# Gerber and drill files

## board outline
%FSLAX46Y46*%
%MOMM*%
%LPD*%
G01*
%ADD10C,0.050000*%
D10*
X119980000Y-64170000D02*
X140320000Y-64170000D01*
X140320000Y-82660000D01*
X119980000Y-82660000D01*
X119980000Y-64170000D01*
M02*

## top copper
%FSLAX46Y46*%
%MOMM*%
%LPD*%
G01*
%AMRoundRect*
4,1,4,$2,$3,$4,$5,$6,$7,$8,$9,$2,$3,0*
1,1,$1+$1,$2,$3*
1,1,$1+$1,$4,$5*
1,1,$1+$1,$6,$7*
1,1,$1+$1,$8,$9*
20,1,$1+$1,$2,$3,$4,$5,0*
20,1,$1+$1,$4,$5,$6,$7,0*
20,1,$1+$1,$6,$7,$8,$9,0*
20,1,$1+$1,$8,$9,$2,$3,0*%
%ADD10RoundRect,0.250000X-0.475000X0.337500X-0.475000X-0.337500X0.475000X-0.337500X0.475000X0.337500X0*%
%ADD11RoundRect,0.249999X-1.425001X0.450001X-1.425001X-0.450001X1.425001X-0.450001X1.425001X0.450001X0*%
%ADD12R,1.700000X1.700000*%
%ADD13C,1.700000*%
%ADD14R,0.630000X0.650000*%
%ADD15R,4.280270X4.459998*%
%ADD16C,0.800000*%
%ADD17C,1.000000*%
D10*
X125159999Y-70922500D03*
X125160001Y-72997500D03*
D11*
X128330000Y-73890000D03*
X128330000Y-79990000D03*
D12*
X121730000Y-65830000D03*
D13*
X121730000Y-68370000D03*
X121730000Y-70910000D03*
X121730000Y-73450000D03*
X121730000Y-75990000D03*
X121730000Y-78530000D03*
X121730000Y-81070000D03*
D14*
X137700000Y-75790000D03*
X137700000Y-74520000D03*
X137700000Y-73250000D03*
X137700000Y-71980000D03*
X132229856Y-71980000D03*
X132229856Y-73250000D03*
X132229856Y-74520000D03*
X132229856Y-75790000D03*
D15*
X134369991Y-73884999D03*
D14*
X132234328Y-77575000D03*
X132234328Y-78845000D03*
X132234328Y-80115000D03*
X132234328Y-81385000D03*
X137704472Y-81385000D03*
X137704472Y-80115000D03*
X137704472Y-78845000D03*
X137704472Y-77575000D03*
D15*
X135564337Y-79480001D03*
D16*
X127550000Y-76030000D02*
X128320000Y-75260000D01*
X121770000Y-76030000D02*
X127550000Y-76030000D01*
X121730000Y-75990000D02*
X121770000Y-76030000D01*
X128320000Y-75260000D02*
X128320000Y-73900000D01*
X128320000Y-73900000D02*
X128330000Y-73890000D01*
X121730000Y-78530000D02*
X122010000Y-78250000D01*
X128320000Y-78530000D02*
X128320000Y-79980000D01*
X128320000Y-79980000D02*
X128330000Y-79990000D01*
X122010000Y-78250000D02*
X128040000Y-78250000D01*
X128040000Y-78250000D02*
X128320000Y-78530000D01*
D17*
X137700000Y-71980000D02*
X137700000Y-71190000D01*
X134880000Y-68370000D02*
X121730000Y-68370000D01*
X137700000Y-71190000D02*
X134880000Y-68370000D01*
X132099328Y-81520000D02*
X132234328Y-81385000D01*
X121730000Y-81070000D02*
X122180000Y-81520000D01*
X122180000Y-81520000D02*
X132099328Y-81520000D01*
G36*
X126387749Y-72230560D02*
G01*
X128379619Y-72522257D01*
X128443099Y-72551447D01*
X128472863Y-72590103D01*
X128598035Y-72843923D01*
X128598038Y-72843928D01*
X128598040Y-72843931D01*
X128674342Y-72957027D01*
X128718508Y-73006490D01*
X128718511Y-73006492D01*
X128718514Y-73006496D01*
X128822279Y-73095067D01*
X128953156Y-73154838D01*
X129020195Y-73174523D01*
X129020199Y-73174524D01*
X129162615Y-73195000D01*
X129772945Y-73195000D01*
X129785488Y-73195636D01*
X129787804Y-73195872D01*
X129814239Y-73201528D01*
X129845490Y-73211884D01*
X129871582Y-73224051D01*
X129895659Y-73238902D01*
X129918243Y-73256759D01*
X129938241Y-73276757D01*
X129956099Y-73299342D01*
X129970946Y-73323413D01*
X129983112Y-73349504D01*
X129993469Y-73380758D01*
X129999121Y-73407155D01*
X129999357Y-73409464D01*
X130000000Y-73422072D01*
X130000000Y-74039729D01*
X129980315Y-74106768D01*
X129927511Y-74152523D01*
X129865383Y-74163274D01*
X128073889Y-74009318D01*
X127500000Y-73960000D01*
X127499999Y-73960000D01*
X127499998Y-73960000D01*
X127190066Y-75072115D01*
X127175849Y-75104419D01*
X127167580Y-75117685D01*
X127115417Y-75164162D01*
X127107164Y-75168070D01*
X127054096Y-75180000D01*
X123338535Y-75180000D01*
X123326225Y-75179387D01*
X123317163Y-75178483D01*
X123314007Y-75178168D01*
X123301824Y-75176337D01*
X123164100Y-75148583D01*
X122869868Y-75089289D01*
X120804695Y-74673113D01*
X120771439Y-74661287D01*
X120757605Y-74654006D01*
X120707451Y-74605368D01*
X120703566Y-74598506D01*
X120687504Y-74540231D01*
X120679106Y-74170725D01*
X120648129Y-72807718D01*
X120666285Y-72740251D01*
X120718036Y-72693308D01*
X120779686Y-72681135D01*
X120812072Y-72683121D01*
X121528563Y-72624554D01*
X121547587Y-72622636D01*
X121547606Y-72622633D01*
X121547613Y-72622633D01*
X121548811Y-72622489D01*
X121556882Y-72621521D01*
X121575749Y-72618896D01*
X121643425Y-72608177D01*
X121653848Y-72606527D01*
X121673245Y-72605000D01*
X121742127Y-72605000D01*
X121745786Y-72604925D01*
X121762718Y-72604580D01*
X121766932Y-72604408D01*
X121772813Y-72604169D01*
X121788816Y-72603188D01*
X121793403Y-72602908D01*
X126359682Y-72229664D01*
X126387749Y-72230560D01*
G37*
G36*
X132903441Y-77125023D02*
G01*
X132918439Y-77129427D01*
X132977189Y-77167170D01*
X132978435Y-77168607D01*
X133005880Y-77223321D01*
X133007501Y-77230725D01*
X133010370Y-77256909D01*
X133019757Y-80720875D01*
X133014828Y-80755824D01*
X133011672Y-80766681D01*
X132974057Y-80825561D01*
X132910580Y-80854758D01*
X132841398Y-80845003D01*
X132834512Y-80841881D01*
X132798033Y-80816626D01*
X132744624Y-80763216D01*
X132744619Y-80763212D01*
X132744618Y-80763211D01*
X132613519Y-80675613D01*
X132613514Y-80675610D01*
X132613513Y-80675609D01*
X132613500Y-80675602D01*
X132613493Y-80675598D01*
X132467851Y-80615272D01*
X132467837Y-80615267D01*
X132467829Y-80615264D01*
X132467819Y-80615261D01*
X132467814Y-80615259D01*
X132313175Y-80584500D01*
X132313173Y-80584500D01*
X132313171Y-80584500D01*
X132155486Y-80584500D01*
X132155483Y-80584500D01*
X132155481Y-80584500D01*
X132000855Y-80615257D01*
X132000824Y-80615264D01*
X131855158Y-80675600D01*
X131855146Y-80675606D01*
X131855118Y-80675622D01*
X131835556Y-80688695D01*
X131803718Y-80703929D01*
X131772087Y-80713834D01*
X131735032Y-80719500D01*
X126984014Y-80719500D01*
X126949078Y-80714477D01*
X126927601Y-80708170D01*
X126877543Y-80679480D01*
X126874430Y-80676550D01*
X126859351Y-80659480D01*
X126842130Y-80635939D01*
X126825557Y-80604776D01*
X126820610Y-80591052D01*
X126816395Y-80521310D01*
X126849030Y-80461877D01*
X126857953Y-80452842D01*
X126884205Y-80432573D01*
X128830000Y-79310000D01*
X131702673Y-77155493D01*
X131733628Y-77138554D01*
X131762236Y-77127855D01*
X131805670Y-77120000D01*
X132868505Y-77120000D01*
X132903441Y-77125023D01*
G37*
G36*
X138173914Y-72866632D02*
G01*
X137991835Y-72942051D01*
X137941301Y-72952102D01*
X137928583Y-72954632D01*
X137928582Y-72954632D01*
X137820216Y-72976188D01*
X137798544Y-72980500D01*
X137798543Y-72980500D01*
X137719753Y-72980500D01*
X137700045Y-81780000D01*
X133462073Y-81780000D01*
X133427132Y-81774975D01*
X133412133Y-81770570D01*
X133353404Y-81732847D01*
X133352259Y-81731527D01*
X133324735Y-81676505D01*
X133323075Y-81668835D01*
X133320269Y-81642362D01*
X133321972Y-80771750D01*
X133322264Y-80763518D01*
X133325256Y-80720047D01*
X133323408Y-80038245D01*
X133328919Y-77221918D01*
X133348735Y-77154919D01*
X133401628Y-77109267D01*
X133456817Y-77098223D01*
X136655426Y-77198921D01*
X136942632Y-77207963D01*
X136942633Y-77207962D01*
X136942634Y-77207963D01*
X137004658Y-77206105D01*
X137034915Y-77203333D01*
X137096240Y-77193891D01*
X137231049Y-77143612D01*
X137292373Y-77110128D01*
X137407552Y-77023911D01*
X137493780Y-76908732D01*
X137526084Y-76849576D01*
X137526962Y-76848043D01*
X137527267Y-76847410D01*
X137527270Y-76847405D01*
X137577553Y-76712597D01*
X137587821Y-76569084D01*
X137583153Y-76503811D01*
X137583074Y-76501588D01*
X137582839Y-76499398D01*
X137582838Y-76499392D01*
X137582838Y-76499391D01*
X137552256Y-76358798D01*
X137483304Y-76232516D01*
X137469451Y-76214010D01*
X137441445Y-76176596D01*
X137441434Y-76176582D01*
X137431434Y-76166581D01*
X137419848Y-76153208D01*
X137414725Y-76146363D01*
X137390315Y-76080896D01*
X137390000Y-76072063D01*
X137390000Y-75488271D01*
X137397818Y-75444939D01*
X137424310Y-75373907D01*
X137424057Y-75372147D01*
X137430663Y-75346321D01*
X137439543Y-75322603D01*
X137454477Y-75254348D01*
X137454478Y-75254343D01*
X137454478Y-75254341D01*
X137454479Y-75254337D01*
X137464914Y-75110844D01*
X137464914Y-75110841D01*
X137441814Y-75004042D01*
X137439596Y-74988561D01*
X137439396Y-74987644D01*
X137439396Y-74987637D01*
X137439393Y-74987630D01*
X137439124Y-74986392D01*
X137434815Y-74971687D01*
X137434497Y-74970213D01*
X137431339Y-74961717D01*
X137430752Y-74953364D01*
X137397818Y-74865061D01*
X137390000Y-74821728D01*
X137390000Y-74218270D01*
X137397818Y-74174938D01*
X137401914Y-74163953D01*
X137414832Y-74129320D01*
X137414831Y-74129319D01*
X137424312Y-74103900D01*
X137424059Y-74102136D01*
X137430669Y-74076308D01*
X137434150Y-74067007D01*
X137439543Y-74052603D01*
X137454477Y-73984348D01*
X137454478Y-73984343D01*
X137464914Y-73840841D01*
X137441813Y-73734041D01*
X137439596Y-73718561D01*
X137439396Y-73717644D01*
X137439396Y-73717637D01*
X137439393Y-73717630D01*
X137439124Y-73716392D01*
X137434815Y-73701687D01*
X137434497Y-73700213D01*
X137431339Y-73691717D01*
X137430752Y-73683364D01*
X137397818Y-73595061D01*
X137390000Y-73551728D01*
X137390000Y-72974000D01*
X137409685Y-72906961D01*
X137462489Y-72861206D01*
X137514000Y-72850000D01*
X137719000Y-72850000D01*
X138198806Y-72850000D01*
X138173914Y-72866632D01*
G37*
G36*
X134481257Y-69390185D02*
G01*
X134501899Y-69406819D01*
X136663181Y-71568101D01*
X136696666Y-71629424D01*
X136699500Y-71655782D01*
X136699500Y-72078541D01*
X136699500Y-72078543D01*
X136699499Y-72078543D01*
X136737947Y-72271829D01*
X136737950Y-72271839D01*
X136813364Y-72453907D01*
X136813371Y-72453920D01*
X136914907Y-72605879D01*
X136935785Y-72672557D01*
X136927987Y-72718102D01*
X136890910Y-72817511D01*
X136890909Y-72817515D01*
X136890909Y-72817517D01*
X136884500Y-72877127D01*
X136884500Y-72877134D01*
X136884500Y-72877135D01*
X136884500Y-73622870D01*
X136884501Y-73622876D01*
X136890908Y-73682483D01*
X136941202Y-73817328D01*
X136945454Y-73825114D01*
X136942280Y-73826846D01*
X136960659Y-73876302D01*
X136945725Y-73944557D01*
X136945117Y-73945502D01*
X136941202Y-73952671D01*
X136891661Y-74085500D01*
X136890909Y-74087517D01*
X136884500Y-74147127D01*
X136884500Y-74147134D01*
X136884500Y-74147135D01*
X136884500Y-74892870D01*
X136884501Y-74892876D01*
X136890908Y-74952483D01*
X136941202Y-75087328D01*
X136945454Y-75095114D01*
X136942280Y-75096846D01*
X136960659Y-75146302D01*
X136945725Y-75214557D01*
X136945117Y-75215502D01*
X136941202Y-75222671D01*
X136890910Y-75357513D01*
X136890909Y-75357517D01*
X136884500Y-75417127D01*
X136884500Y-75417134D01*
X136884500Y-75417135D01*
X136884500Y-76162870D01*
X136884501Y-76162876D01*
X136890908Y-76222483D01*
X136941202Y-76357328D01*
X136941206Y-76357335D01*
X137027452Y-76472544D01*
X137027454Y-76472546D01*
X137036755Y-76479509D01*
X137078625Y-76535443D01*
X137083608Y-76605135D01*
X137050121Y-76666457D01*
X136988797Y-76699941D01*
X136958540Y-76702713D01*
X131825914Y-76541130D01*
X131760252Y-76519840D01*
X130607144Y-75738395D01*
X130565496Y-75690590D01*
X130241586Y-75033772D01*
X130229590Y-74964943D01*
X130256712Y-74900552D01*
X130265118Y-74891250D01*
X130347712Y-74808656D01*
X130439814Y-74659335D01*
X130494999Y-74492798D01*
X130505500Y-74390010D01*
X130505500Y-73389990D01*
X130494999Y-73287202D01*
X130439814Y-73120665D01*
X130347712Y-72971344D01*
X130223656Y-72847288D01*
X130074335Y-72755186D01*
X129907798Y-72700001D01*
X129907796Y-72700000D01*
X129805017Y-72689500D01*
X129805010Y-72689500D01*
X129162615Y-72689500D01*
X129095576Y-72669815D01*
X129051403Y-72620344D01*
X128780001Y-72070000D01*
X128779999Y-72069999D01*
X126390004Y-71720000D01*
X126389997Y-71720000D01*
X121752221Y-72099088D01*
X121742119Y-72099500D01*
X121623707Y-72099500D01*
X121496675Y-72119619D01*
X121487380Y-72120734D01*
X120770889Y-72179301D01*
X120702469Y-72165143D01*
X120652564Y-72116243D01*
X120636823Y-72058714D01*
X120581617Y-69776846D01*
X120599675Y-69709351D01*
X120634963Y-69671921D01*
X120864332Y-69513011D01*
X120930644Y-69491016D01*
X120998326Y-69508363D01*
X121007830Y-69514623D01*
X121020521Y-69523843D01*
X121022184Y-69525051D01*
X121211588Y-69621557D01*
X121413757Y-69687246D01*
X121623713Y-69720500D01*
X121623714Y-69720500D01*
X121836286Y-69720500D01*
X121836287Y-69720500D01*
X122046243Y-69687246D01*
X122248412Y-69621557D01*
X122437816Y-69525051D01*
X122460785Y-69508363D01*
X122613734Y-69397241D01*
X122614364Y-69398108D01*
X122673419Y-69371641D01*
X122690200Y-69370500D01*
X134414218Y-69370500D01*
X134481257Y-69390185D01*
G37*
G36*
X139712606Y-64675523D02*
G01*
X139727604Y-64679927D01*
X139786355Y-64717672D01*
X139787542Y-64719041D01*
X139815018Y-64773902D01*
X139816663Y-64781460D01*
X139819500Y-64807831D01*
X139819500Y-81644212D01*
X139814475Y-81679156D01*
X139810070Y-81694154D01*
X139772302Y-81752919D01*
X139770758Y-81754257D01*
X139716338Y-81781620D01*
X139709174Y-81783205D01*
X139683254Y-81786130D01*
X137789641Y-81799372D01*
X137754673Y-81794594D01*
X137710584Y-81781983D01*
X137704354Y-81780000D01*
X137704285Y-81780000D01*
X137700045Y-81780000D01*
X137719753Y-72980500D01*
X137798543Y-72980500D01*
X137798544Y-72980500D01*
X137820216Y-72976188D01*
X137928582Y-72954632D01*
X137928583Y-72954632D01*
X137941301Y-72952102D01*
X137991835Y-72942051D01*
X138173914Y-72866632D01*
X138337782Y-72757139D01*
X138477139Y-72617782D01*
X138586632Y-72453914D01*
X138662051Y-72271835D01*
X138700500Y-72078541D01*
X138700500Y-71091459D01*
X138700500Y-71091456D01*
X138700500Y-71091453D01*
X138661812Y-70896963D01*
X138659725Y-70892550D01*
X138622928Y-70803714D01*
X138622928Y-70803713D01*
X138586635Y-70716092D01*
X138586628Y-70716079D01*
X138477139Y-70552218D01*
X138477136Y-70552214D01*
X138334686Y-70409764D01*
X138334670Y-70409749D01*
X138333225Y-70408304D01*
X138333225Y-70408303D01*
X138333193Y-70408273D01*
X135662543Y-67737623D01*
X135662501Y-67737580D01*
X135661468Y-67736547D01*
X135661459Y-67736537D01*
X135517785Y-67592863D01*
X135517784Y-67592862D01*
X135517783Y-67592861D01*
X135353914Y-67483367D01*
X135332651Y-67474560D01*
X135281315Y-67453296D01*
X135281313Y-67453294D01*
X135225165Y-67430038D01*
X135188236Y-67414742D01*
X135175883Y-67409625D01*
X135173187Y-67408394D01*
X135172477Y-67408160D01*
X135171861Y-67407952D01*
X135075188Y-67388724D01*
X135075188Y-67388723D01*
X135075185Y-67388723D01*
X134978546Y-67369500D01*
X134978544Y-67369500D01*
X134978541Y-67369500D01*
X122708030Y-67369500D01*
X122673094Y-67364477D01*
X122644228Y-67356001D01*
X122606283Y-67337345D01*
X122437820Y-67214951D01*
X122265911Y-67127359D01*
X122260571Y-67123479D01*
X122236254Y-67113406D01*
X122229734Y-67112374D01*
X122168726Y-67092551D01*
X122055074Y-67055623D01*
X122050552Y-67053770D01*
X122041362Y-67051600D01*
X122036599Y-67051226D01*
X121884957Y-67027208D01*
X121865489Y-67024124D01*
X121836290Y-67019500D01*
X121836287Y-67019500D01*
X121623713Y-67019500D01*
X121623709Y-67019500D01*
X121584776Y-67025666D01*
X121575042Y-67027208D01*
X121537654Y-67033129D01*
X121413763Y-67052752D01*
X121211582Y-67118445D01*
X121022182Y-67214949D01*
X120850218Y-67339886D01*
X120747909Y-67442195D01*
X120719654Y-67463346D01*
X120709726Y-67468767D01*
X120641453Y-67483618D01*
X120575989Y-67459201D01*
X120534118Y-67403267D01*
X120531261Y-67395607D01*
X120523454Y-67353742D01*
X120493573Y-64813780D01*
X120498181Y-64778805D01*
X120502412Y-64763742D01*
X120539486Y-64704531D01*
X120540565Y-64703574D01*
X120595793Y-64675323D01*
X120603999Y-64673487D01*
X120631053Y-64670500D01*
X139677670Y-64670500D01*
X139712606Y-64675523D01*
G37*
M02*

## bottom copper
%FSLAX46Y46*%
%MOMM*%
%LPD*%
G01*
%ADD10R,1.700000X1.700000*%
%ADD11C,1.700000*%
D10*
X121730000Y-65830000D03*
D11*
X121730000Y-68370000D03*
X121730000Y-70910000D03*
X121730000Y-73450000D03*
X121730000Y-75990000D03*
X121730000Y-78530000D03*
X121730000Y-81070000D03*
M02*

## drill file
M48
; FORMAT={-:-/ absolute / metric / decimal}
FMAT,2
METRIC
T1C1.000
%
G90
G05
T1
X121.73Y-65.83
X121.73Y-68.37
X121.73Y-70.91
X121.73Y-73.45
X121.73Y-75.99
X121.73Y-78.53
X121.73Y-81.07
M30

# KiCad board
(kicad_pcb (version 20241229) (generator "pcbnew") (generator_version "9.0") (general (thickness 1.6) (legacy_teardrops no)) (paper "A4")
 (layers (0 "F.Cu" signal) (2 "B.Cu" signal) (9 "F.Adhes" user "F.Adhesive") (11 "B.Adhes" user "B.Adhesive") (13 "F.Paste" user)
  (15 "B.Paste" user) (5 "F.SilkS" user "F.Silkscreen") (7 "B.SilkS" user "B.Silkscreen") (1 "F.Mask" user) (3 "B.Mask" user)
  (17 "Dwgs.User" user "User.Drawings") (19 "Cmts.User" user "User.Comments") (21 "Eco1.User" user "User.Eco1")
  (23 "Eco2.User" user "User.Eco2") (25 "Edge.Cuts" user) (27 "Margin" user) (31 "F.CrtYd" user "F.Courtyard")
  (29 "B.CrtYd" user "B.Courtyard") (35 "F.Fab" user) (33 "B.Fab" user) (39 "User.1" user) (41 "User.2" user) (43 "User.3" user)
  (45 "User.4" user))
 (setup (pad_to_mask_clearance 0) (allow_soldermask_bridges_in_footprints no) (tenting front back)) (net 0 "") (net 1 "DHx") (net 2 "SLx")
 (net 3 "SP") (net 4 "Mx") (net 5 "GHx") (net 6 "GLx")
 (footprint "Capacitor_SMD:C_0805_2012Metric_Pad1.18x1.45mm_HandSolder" (layer "F.Cu") (at 125.16 71.96 -90)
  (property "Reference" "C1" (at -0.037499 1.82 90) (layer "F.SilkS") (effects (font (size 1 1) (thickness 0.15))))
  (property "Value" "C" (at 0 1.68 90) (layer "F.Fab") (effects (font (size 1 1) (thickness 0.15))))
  (pad "1" smd roundrect (at -1.0375 0.000001 270) (size 1.175 1.45) (layers "F.Cu" "F.Mask" "F.Paste") (roundrect_rratio 0.212766)
   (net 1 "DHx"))
  (pad "2" smd roundrect (at 1.0375 -0.000001 270) (size 1.175 1.45) (layers "F.Cu" "F.Mask" "F.Paste") (roundrect_rratio 0.212766)
   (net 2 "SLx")))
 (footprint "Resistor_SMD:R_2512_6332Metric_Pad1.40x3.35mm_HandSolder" (layer "F.Cu") (at 128.33 76.94 -90)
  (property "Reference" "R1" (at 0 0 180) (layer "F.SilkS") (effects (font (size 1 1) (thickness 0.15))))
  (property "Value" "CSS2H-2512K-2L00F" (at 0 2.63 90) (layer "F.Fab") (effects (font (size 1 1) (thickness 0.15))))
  (pad "1" smd roundrect (at -3.05 0 270) (size 1.4 3.35) (layers "F.Cu" "F.Mask" "F.Paste") (roundrect_rratio 0.178571) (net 2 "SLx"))
  (pad "2" smd roundrect (at 3.05 0 270) (size 1.4 3.35) (layers "F.Cu" "F.Mask" "F.Paste") (roundrect_rratio 0.178571) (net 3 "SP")))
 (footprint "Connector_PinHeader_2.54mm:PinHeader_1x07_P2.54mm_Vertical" (layer "F.Cu") (at 121.73 65.83)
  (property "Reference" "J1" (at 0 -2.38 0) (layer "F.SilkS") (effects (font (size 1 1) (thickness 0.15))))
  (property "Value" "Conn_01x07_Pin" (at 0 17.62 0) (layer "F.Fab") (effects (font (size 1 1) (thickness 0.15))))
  (pad "1" thru_hole rect (at 0 0) (size 1.7 1.7) (drill 1) (layers "*.Cu" "*.Mask") (remove_unused_layers no) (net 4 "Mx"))
  (pad "2" thru_hole circle (at 0 2.54) (size 1.7 1.7) (drill 1) (layers "*.Cu" "*.Mask") (remove_unused_layers no) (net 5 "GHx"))
  (pad "3" thru_hole circle (at 0 5.08) (size 1.7 1.7) (drill 1) (layers "*.Cu" "*.Mask") (remove_unused_layers no) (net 1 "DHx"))
  (pad "4" thru_hole circle (at 0 7.62) (size 1.7 1.7) (drill 1) (layers "*.Cu" "*.Mask") (remove_unused_layers no) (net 2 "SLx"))
  (pad "5" thru_hole circle (at 0 10.16) (size 1.7 1.7) (drill 1) (layers "*.Cu" "*.Mask") (remove_unused_layers no) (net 2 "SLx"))
  (pad "6" thru_hole circle (at 0 12.7) (size 1.7 1.7) (drill 1) (layers "*.Cu" "*.Mask") (remove_unused_layers no) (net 3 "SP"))
  (pad "7" thru_hole circle (at 0 15.24) (size 1.7 1.7) (drill 1) (layers "*.Cu" "*.Mask") (remove_unused_layers no) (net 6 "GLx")))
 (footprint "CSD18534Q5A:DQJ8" (layer "F.Cu") (at 134.964928 73.885 180)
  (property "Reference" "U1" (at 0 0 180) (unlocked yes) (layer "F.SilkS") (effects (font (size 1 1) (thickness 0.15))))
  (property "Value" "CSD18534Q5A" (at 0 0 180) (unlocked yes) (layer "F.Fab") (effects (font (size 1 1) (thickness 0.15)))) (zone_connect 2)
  (pad "1" smd rect (at -2.735072 -1.905 180) (size 0.63 0.65) (layers "F.Cu" "F.Mask" "F.Paste") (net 4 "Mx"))
  (pad "2" smd rect (at -2.735072 -0.635 180) (size 0.63 0.65) (layers "F.Cu" "F.Mask" "F.Paste") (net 4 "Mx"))
  (pad "3" smd rect (at -2.735072 0.635 180) (size 0.63 0.65) (layers "F.Cu" "F.Mask" "F.Paste") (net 4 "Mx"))
  (pad "4" smd rect (at -2.735072 1.905 180) (size 0.63 0.65) (layers "F.Cu" "F.Mask" "F.Paste") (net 5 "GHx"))
  (pad "5" smd rect (at 2.735072 1.905 180) (size 0.63 0.65) (layers "F.Cu" "F.Mask" "F.Paste") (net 1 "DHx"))
  (pad "6" smd rect (at 2.735072 0.635 180) (size 0.63 0.65) (layers "F.Cu" "F.Mask" "F.Paste") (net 1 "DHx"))
  (pad "7" smd rect (at 2.735072 -0.635 180) (size 0.63 0.65) (layers "F.Cu" "F.Mask" "F.Paste") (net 1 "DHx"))
  (pad "8" smd rect (at 2.735072 -1.905 180) (size 0.63 0.65) (layers "F.Cu" "F.Mask" "F.Paste") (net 1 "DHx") (clearance 0)
   (zone_connect 2) (thermal_bridge_width 0.25) (thermal_gap 0.25))
  (pad "9" smd rect (at 0.594937 0.000001 180) (size 4.28027 4.459998) (layers "F.Cu" "F.Mask" "F.Paste") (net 1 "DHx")))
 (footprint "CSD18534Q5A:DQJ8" (layer "F.Cu") (at 134.9694 79.48)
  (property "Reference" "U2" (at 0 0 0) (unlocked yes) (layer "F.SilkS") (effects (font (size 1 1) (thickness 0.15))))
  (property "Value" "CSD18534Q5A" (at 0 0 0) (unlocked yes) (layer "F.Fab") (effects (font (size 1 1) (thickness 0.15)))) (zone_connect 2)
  (pad "1" smd rect (at -2.735072 -1.905) (size 0.63 0.65) (layers "F.Cu" "F.Mask" "F.Paste") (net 3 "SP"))
  (pad "2" smd rect (at -2.735072 -0.635) (size 0.63 0.65) (layers "F.Cu" "F.Mask" "F.Paste") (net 3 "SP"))
  (pad "3" smd rect (at -2.735072 0.635) (size 0.63 0.65) (layers "F.Cu" "F.Mask" "F.Paste") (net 3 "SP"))
  (pad "4" smd rect (at -2.735072 1.905) (size 0.63 0.65) (layers "F.Cu" "F.Mask" "F.Paste") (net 6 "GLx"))
  (pad "5" smd rect (at 2.735072 1.905) (size 0.63 0.65) (layers "F.Cu" "F.Mask" "F.Paste") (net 4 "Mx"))
  (pad "6" smd rect (at 2.735072 0.635) (size 0.63 0.65) (layers "F.Cu" "F.Mask" "F.Paste") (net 4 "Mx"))
  (pad "7" smd rect (at 2.735072 -0.635) (size 0.63 0.65) (layers "F.Cu" "F.Mask" "F.Paste") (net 4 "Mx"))
  (pad "8" smd rect (at 2.735072 -1.905) (size 0.63 0.65) (layers "F.Cu" "F.Mask" "F.Paste") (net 4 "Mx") (clearance 0) (zone_connect 2)
   (thermal_bridge_width 0.25) (thermal_gap 0.25))
  (pad "9" smd rect (at 0.594937 0.000001) (size 4.28027 4.459998) (layers "F.Cu" "F.Mask" "F.Paste") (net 4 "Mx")))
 (gr_rect (start 119.98 64.17) (end 140.32 82.66) (stroke (width 0.05) (type default)) (fill no) (layer "Edge.Cuts"))
 (segment (start 127.55 76.03) (end 128.32 75.26) (width 0.8) (layer "F.Cu") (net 2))
 (segment (start 121.77 76.03) (end 127.55 76.03) (width 0.8) (layer "F.Cu") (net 2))
 (segment (start 121.73 75.99) (end 121.77 76.03) (width 0.8) (layer "F.Cu") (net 2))
 (segment (start 128.32 75.26) (end 128.32 73.9) (width 0.8) (layer "F.Cu") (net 2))
 (segment (start 128.32 73.9) (end 128.33 73.89) (width 0.8) (layer "F.Cu") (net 2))
 (segment (start 121.73 78.53) (end 122.01 78.25) (width 0.8) (layer "F.Cu") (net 3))
 (segment (start 128.32 78.53) (end 128.32 79.98) (width 0.8) (layer "F.Cu") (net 3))
 (segment (start 128.32 79.98) (end 128.33 79.99) (width 0.8) (layer "F.Cu") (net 3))
 (segment (start 122.01 78.25) (end 128.04 78.25) (width 0.8) (layer "F.Cu") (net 3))
 (segment (start 128.04 78.25) (end 128.32 78.53) (width 0.8) (layer "F.Cu") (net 3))
 (segment (start 137.7 71.98) (end 137.7 71.19) (width 1) (layer "F.Cu") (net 5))
 (segment (start 134.88 68.37) (end 121.73 68.37) (width 1) (layer "F.Cu") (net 5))
 (segment (start 137.7 71.19) (end 134.88 68.37) (width 1) (layer "F.Cu") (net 5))
 (segment (start 132.099328 81.52) (end 132.234328 81.385) (width 1) (layer "F.Cu") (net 6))
 (segment (start 121.73 81.07) (end 122.18 81.52) (width 1) (layer "F.Cu") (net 6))
 (segment (start 122.18 81.52) (end 132.099328 81.52) (width 1) (layer "F.Cu") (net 6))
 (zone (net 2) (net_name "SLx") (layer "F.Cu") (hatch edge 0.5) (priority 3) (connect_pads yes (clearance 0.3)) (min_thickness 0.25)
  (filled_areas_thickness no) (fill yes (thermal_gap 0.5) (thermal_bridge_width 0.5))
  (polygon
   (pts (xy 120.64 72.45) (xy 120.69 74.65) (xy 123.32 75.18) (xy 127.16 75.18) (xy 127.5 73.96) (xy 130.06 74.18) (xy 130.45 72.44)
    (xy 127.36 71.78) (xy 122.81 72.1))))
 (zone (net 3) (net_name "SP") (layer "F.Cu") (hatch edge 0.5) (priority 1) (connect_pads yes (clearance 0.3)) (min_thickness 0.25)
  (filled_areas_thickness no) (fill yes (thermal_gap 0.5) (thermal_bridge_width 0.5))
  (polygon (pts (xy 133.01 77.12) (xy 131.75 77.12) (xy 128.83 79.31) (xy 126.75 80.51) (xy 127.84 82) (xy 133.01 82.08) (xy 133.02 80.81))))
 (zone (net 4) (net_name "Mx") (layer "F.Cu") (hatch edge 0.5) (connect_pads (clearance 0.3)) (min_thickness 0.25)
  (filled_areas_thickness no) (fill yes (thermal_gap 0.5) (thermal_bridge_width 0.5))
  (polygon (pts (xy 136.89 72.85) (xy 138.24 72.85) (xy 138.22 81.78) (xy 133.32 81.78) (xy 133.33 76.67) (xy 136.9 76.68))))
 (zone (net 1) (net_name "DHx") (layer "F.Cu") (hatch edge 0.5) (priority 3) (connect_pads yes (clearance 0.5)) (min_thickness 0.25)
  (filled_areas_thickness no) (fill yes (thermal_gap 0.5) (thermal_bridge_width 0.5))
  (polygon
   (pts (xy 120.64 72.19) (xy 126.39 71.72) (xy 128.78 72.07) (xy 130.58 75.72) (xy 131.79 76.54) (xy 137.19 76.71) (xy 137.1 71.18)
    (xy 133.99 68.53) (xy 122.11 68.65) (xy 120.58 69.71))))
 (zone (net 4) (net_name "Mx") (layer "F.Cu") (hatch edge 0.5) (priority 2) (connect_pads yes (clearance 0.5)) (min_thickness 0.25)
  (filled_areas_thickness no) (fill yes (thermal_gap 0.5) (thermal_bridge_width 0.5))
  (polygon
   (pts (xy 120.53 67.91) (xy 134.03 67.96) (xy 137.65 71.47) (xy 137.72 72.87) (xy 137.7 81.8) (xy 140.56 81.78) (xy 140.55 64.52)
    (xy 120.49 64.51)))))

